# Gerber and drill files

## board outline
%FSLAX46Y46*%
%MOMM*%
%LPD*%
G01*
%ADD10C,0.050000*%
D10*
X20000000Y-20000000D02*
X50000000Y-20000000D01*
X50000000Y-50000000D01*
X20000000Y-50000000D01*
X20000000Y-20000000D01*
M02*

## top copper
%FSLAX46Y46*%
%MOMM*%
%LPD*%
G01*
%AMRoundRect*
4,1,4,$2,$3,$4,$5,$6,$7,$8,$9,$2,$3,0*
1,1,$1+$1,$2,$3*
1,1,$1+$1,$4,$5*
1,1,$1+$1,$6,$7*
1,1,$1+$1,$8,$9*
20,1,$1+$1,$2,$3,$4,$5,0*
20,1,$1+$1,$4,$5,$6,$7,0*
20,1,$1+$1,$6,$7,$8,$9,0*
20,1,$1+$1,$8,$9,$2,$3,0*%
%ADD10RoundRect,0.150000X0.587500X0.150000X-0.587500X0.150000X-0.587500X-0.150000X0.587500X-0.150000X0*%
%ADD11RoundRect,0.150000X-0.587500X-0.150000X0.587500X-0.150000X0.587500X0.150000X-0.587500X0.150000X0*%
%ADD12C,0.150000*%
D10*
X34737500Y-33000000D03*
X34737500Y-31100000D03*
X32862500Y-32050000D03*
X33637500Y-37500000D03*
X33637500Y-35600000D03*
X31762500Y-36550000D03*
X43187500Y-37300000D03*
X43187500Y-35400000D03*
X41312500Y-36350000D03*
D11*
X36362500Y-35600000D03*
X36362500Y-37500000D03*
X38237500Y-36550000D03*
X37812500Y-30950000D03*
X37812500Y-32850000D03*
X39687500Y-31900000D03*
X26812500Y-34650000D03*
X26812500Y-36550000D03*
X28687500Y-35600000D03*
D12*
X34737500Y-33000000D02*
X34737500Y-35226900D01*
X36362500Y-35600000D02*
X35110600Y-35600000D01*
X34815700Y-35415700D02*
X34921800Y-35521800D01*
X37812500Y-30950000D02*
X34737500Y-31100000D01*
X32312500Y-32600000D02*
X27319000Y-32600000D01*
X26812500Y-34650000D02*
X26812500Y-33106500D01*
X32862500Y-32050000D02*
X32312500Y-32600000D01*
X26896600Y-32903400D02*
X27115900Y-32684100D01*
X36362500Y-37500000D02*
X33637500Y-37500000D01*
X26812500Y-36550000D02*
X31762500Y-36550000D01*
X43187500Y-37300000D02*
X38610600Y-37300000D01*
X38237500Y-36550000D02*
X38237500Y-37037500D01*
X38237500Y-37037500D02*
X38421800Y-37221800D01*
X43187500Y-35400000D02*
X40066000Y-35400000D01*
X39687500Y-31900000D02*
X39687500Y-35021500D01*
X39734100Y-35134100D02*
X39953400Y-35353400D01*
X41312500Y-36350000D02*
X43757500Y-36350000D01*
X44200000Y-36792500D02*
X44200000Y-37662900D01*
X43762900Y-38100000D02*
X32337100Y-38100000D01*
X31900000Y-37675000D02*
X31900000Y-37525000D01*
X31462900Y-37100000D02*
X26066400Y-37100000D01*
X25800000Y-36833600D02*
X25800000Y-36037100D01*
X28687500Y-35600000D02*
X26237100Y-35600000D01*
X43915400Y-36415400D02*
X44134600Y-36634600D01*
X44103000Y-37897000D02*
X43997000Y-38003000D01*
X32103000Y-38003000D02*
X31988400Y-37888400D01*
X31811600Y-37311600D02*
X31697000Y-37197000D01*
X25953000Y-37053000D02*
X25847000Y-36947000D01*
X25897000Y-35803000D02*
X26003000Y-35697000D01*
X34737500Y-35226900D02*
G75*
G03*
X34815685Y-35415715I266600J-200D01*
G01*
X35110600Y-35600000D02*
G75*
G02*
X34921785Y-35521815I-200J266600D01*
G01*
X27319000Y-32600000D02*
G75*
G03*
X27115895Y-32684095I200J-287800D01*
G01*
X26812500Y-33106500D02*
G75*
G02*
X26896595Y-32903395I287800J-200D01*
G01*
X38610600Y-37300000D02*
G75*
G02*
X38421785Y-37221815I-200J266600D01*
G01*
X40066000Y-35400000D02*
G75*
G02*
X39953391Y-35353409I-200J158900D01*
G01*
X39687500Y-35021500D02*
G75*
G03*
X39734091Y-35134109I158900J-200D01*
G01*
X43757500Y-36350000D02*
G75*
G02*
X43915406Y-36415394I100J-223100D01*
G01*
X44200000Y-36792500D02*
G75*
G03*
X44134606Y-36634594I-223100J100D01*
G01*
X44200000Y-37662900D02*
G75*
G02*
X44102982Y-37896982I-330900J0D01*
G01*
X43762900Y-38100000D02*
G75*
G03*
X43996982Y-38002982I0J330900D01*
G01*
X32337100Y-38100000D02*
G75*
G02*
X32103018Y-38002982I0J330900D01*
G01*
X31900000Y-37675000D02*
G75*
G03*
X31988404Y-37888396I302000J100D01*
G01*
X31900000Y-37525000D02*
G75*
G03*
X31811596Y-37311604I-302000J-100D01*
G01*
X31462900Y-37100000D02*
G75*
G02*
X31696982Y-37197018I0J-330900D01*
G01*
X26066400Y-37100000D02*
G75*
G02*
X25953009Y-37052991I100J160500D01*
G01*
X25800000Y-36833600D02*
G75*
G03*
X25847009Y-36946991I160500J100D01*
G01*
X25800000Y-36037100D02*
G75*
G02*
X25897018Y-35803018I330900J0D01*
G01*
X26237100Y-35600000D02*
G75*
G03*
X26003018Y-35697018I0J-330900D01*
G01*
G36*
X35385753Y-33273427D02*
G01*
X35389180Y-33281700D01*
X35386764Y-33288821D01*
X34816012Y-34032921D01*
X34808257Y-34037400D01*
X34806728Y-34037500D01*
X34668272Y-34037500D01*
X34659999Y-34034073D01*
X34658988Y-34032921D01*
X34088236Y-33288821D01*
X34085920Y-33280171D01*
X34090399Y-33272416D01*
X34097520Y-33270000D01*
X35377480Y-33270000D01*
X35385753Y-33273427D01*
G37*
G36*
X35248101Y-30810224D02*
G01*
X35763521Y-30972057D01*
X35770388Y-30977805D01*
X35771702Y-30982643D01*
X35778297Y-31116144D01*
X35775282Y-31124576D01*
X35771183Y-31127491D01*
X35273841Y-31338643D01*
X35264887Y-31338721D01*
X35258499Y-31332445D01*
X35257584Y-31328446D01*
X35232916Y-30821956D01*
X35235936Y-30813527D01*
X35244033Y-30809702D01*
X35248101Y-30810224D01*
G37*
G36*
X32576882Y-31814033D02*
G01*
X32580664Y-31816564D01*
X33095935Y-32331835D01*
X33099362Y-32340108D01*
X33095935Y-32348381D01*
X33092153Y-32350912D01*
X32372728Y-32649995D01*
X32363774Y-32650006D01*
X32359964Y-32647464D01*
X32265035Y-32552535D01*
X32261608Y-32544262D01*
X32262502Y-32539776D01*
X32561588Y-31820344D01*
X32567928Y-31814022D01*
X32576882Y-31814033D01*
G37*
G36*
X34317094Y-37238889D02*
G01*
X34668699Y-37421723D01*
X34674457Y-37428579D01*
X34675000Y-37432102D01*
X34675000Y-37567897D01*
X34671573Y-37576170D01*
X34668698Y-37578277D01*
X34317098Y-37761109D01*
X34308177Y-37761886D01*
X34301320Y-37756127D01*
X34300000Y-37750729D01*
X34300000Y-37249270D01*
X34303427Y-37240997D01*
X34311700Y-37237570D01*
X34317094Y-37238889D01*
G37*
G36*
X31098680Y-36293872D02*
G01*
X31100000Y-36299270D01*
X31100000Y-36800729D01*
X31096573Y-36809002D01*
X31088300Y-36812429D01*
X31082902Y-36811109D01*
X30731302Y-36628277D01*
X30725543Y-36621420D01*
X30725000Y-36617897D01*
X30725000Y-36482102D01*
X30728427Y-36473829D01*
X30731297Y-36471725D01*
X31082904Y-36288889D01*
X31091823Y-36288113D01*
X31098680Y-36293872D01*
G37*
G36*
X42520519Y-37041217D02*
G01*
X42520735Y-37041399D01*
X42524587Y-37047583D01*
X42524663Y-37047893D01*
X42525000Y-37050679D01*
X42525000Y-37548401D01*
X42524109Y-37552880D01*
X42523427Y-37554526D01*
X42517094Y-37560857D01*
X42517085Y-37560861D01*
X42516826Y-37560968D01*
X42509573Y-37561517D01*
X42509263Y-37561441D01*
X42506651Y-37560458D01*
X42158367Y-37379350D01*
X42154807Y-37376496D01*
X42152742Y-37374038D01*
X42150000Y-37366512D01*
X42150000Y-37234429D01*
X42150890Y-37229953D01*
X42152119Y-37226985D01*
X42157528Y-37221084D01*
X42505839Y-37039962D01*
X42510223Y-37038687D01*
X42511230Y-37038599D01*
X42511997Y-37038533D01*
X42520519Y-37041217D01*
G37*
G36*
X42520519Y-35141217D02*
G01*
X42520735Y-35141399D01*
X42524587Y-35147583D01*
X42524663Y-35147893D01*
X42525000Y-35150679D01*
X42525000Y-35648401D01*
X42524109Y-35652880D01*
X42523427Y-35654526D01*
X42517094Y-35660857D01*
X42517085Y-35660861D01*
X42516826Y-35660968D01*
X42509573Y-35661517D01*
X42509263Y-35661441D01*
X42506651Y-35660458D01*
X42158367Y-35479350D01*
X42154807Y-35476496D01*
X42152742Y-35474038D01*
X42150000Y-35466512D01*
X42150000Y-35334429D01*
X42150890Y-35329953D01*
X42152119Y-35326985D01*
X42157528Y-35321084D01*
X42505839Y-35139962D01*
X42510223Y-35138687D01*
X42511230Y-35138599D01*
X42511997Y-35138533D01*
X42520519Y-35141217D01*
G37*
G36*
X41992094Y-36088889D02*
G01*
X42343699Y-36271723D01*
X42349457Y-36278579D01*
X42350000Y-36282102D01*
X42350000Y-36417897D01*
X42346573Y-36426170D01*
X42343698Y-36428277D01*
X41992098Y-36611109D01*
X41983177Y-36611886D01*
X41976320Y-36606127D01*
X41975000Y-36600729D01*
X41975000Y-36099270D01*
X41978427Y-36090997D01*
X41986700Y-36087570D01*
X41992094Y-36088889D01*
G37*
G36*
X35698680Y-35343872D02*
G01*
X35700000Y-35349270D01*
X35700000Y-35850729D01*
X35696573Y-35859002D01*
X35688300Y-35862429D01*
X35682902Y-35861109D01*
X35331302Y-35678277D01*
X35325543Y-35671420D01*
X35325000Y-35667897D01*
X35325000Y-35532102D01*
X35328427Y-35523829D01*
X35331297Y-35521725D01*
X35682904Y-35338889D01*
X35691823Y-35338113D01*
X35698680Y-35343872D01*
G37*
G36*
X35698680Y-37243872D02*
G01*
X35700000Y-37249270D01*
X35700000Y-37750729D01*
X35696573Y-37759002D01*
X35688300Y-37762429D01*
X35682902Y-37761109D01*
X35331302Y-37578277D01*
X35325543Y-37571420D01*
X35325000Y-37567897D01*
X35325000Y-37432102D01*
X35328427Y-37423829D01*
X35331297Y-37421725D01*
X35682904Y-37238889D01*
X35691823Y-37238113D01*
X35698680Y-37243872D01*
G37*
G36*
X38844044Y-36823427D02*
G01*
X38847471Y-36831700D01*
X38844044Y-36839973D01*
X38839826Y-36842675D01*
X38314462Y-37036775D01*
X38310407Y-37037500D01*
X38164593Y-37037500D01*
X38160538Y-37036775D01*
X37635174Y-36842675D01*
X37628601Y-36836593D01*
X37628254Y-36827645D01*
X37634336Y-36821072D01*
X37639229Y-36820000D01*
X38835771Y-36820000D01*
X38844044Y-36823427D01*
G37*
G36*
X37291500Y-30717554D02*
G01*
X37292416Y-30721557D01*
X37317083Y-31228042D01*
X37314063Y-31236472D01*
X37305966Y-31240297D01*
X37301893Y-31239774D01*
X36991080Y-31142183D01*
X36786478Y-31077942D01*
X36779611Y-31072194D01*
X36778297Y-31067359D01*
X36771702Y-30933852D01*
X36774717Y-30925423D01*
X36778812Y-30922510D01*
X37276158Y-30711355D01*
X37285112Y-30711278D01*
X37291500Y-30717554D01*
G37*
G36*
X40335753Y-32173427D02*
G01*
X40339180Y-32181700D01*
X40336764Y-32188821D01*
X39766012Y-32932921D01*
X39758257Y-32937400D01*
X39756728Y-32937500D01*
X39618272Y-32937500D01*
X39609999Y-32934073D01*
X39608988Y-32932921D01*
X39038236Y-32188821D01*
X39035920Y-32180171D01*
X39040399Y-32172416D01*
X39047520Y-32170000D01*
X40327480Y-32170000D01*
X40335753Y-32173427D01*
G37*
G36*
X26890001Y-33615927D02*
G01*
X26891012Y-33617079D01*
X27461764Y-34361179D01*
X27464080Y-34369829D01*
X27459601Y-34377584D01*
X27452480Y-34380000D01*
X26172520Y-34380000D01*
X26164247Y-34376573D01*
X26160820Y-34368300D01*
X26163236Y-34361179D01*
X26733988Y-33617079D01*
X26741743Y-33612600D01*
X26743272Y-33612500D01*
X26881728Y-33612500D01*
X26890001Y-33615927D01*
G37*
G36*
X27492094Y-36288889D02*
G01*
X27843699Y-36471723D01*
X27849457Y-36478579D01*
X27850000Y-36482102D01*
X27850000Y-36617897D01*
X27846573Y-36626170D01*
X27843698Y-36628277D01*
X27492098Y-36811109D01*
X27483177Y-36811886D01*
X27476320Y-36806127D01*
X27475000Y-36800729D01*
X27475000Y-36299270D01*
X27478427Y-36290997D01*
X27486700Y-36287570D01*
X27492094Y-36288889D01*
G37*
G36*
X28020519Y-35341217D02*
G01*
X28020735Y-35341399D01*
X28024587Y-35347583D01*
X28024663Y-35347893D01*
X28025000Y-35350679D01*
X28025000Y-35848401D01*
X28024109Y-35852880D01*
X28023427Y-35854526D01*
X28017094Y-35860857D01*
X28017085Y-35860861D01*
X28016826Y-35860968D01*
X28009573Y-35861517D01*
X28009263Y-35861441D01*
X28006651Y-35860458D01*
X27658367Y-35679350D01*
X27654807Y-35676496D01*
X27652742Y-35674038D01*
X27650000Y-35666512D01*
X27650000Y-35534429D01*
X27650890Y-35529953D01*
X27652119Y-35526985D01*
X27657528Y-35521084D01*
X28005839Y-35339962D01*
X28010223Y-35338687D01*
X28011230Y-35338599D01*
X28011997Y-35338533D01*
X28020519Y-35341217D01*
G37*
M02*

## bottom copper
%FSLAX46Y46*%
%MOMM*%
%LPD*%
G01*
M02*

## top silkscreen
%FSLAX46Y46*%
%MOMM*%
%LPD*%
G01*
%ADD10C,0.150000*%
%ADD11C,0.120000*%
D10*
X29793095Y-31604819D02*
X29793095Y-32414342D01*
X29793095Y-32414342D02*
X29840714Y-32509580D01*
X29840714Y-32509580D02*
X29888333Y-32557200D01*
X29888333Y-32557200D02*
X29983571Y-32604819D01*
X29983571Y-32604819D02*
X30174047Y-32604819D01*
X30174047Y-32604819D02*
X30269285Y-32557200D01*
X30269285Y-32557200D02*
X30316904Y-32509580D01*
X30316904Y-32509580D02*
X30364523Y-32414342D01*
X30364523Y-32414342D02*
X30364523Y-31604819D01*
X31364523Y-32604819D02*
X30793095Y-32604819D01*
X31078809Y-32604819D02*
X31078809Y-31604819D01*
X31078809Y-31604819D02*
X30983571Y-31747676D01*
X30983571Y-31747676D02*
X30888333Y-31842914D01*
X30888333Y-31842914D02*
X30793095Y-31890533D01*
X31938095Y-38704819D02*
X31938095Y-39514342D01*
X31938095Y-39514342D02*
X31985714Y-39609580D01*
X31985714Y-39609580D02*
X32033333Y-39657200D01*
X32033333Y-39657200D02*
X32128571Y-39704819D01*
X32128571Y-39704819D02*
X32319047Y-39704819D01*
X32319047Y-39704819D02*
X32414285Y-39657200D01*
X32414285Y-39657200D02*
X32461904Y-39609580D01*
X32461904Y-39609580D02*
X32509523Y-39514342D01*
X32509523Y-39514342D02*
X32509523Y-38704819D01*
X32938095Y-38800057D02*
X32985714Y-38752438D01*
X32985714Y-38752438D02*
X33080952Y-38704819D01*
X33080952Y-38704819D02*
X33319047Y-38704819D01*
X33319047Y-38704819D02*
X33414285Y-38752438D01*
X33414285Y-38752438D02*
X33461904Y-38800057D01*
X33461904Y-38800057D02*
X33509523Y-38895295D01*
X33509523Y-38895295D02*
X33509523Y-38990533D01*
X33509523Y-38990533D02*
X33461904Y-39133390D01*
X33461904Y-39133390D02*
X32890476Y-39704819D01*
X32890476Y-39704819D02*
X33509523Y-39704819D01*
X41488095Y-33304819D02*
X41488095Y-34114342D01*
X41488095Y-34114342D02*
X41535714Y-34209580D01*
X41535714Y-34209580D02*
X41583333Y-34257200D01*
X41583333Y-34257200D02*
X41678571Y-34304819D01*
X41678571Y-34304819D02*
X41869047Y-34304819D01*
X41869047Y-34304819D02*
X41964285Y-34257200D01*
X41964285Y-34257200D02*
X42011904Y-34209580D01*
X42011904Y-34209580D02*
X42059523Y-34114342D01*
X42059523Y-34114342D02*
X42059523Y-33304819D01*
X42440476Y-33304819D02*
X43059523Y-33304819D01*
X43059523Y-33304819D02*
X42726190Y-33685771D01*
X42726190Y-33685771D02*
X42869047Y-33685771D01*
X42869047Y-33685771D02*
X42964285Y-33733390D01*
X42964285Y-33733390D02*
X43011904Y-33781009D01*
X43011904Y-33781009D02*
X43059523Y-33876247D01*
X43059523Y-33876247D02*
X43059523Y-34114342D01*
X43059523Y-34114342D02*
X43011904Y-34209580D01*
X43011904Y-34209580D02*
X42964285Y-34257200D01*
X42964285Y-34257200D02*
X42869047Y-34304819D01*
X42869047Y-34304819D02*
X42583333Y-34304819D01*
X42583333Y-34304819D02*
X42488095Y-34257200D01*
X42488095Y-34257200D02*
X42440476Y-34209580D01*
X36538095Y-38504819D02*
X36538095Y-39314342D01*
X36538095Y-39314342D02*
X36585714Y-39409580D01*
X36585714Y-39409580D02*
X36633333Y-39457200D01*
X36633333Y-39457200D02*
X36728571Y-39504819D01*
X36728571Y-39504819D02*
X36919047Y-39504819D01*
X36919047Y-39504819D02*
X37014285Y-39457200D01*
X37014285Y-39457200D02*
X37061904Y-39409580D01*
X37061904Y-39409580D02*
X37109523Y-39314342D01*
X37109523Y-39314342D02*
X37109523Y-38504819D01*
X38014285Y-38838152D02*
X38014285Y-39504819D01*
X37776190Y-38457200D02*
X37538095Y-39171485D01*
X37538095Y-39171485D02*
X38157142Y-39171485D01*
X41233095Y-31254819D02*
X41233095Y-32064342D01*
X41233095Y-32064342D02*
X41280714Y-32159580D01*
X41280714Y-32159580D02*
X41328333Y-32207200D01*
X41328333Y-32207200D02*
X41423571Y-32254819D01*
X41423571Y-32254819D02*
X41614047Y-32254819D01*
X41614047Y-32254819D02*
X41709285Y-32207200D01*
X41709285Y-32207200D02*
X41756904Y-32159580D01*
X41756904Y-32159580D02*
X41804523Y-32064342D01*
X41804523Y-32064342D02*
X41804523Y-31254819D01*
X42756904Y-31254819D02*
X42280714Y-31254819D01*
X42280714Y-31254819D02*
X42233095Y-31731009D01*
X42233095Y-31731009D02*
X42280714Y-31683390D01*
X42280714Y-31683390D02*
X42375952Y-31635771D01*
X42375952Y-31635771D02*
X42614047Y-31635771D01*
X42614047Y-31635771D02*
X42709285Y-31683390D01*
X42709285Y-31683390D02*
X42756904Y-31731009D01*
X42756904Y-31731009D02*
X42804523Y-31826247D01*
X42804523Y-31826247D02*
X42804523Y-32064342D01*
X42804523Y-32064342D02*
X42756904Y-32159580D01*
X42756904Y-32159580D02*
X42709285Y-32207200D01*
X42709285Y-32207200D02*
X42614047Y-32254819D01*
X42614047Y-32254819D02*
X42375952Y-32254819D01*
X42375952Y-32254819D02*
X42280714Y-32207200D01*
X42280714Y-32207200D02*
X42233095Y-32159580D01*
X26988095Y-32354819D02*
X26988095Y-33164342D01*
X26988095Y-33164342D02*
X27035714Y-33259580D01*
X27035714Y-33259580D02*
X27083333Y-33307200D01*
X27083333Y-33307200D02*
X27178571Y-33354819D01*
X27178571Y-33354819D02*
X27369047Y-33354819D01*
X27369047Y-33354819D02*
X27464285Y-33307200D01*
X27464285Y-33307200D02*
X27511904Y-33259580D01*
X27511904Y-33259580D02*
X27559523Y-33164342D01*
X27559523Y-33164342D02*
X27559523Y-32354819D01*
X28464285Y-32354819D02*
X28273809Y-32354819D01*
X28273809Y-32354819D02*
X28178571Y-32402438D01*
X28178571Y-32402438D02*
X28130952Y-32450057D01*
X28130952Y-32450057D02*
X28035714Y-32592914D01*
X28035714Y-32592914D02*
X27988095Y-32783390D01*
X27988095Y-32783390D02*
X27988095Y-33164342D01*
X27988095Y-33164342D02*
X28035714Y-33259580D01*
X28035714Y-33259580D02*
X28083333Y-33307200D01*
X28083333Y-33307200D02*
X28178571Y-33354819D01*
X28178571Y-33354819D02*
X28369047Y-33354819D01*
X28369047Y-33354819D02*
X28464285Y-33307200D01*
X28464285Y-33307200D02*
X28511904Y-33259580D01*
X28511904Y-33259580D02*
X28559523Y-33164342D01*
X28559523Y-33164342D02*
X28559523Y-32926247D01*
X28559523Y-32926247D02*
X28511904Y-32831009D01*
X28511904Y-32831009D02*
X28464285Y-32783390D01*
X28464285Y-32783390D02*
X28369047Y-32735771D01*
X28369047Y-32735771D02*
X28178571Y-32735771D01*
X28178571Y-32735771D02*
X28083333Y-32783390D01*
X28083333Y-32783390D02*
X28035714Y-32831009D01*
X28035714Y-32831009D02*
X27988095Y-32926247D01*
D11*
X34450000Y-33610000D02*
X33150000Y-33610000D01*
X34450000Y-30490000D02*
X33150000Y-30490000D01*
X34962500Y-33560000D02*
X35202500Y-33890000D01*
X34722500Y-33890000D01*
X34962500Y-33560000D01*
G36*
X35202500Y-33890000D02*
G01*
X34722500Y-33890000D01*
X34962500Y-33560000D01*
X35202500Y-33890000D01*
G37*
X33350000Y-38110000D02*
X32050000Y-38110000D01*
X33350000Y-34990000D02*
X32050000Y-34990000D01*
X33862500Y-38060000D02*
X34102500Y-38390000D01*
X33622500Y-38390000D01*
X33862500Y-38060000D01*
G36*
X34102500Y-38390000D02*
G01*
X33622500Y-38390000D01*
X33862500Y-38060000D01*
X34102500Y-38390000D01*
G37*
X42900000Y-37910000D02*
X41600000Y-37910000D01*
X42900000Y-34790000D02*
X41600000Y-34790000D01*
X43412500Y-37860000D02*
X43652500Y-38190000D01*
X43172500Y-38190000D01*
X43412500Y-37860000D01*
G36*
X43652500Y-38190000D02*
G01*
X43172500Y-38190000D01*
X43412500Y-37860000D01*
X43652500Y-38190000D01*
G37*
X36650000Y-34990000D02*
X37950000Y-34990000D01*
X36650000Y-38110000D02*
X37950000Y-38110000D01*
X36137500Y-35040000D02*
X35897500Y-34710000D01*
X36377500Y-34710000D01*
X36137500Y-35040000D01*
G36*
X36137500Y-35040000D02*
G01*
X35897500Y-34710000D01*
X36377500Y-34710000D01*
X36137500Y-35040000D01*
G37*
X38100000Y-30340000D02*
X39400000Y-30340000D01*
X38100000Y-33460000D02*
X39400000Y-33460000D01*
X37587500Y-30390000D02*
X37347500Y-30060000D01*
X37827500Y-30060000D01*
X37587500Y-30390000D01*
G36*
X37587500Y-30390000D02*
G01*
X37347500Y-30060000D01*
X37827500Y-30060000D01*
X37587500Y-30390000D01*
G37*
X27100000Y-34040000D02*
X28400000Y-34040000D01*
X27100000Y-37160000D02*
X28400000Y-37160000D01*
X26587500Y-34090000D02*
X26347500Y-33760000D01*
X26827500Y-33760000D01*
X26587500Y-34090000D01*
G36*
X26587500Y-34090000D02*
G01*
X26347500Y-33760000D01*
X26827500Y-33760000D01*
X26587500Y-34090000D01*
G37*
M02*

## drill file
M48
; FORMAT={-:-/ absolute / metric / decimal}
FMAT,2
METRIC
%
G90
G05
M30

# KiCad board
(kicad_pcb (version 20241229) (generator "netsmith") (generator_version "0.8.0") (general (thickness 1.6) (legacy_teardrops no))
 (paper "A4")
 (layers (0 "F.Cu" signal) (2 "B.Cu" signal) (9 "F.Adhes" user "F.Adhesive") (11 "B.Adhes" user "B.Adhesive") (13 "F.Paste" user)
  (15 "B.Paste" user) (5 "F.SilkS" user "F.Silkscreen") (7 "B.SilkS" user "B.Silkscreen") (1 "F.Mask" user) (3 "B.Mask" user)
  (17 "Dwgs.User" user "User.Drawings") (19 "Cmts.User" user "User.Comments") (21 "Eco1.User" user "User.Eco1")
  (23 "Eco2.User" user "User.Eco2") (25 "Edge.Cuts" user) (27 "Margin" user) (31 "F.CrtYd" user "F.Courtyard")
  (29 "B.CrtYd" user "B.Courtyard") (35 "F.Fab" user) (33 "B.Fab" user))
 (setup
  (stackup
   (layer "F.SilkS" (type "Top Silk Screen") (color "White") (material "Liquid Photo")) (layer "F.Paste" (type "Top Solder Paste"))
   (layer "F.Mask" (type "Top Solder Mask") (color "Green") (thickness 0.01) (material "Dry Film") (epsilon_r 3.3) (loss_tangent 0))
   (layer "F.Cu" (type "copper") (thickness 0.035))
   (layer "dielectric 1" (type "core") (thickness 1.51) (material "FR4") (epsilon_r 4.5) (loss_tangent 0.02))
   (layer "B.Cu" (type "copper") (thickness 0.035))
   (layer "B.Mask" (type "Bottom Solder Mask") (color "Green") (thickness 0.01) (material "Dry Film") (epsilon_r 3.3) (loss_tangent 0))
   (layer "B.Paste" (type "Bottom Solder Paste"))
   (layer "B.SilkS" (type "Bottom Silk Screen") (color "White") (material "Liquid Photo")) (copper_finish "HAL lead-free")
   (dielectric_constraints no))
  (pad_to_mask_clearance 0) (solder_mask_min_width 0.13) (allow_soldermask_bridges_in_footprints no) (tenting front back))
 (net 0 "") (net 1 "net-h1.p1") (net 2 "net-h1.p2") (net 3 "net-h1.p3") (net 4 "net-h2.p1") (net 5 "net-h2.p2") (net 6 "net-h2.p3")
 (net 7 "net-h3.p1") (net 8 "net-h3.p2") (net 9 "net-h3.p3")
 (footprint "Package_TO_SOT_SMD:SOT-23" (layer "F.Cu") (at 33.8 32.05 180)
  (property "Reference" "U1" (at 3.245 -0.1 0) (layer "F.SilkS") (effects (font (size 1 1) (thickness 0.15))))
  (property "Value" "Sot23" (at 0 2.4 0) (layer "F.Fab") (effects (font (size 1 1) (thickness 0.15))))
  (pad "1" smd roundrect (at -0.9375 -0.95 180) (size 1.475 0.6) (layers "F.Cu" "F.Mask" "F.Paste") (roundrect_rratio 0.25)
   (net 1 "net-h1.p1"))
  (pad "2" smd roundrect (at -0.9375 0.95 180) (size 1.475 0.6) (layers "F.Cu" "F.Mask" "F.Paste") (roundrect_rratio 0.25)
   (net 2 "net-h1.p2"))
  (pad "3" smd roundrect (at 0.9375 0 180) (size 1.475 0.6) (layers "F.Cu" "F.Mask" "F.Paste") (roundrect_rratio 0.25) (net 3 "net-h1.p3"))
  (fp_line (start -0.65 -1.56) (end 0.65 -1.56) (stroke (width 0.12) (type solid)) (layer "F.SilkS"))
  (fp_line (start -0.65 1.56) (end 0.65 1.56) (stroke (width 0.12) (type solid)) (layer "F.SilkS"))
  (fp_poly (pts (xy -1.1625 -1.51) (xy -1.4025 -1.84) (xy -0.9225 -1.84)) (stroke (width 0.12) (type solid)) (fill solid) (layer "F.SilkS")))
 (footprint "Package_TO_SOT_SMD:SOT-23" (layer "F.Cu") (at 32.7 36.55 180)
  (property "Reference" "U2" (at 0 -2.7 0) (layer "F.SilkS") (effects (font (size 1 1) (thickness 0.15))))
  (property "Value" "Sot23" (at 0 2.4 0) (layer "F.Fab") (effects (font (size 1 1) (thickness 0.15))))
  (pad "1" smd roundrect (at -0.9375 -0.95 180) (size 1.475 0.6) (layers "F.Cu" "F.Mask" "F.Paste") (roundrect_rratio 0.25)
   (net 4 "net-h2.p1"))
  (pad "2" smd roundrect (at -0.9375 0.95 180) (size 1.475 0.6) (layers "F.Cu" "F.Mask" "F.Paste") (roundrect_rratio 0.25)
   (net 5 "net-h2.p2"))
  (pad "3" smd roundrect (at 0.9375 0 180) (size 1.475 0.6) (layers "F.Cu" "F.Mask" "F.Paste") (roundrect_rratio 0.25) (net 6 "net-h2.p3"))
  (fp_line (start -0.65 -1.56) (end 0.65 -1.56) (stroke (width 0.12) (type solid)) (layer "F.SilkS"))
  (fp_line (start -0.65 1.56) (end 0.65 1.56) (stroke (width 0.12) (type solid)) (layer "F.SilkS"))
  (fp_poly (pts (xy -1.1625 -1.51) (xy -1.4025 -1.84) (xy -0.9225 -1.84)) (stroke (width 0.12) (type solid)) (fill solid) (layer "F.SilkS")))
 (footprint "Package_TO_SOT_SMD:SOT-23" (layer "F.Cu") (at 42.25 36.35 180)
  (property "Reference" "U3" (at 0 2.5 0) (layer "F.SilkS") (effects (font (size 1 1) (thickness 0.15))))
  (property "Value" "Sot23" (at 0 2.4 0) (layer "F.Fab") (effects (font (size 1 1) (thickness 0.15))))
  (pad "1" smd roundrect (at -0.9375 -0.95 180) (size 1.475 0.6) (layers "F.Cu" "F.Mask" "F.Paste") (roundrect_rratio 0.25)
   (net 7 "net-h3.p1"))
  (pad "2" smd roundrect (at -0.9375 0.95 180) (size 1.475 0.6) (layers "F.Cu" "F.Mask" "F.Paste") (roundrect_rratio 0.25)
   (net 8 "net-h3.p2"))
  (pad "3" smd roundrect (at 0.9375 0 180) (size 1.475 0.6) (layers "F.Cu" "F.Mask" "F.Paste") (roundrect_rratio 0.25) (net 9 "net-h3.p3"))
  (fp_line (start -0.65 -1.56) (end 0.65 -1.56) (stroke (width 0.12) (type solid)) (layer "F.SilkS"))
  (fp_line (start -0.65 1.56) (end 0.65 1.56) (stroke (width 0.12) (type solid)) (layer "F.SilkS"))
  (fp_poly (pts (xy -1.1625 -1.51) (xy -1.4025 -1.84) (xy -0.9225 -1.84)) (stroke (width 0.12) (type solid)) (fill solid) (layer "F.SilkS")))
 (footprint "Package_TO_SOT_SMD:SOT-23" (layer "F.Cu") (at 37.3 36.55)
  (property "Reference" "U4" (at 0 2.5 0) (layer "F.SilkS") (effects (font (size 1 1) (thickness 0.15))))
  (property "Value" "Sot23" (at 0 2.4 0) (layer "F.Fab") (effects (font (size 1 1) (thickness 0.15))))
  (pad "1" smd roundrect (at -0.9375 -0.95) (size 1.475 0.6) (layers "F.Cu" "F.Mask" "F.Paste") (roundrect_rratio 0.25) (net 1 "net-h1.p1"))
  (pad "2" smd roundrect (at -0.9375 0.95) (size 1.475 0.6) (layers "F.Cu" "F.Mask" "F.Paste") (roundrect_rratio 0.25) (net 4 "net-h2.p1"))
  (pad "3" smd roundrect (at 0.9375 0) (size 1.475 0.6) (layers "F.Cu" "F.Mask" "F.Paste") (roundrect_rratio 0.25) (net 7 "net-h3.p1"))
  (fp_line (start -0.65 -1.56) (end 0.65 -1.56) (stroke (width 0.12) (type solid)) (layer "F.SilkS"))
  (fp_line (start -0.65 1.56) (end 0.65 1.56) (stroke (width 0.12) (type solid)) (layer "F.SilkS"))
  (fp_poly (pts (xy -1.1625 -1.51) (xy -1.4025 -1.84) (xy -0.9225 -1.84)) (stroke (width 0.12) (type solid)) (fill solid) (layer "F.SilkS")))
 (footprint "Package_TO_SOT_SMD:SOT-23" (layer "F.Cu") (at 38.75 31.9)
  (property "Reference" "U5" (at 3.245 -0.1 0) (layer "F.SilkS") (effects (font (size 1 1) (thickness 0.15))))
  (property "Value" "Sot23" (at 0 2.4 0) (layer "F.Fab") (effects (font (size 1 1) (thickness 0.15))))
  (pad "1" smd roundrect (at -0.9375 -0.95) (size 1.475 0.6) (layers "F.Cu" "F.Mask" "F.Paste") (roundrect_rratio 0.25) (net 2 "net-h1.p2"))
  (pad "2" smd roundrect (at -0.9375 0.95) (size 1.475 0.6) (layers "F.Cu" "F.Mask" "F.Paste") (roundrect_rratio 0.25) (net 5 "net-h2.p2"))
  (pad "3" smd roundrect (at 0.9375 0) (size 1.475 0.6) (layers "F.Cu" "F.Mask" "F.Paste") (roundrect_rratio 0.25) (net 8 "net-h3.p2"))
  (fp_line (start -0.65 -1.56) (end 0.65 -1.56) (stroke (width 0.12) (type solid)) (layer "F.SilkS"))
  (fp_line (start -0.65 1.56) (end 0.65 1.56) (stroke (width 0.12) (type solid)) (layer "F.SilkS"))
  (fp_poly (pts (xy -1.1625 -1.51) (xy -1.4025 -1.84) (xy -0.9225 -1.84)) (stroke (width 0.12) (type solid)) (fill solid) (layer "F.SilkS")))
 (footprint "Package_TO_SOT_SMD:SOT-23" (layer "F.Cu") (at 27.75 35.6)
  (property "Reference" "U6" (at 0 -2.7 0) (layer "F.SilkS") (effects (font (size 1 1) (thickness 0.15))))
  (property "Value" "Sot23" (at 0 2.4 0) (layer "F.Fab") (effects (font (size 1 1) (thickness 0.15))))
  (pad "1" smd roundrect (at -0.9375 -0.95) (size 1.475 0.6) (layers "F.Cu" "F.Mask" "F.Paste") (roundrect_rratio 0.25) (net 3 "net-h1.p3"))
  (pad "2" smd roundrect (at -0.9375 0.95) (size 1.475 0.6) (layers "F.Cu" "F.Mask" "F.Paste") (roundrect_rratio 0.25) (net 6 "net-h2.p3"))
  (pad "3" smd roundrect (at 0.9375 0) (size 1.475 0.6) (layers "F.Cu" "F.Mask" "F.Paste") (roundrect_rratio 0.25) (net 9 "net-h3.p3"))
  (fp_line (start -0.65 -1.56) (end 0.65 -1.56) (stroke (width 0.12) (type solid)) (layer "F.SilkS"))
  (fp_line (start -0.65 1.56) (end 0.65 1.56) (stroke (width 0.12) (type solid)) (layer "F.SilkS"))
  (fp_poly (pts (xy -1.1625 -1.51) (xy -1.4025 -1.84) (xy -0.9225 -1.84)) (stroke (width 0.12) (type solid)) (fill solid) (layer "F.SilkS")))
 (segment (start 34.7375 33) (end 34.7375 35.2269) (width 0.15) (layer "F.Cu") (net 1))
 (segment (start 36.3625 35.6) (end 35.1106 35.6) (width 0.15) (layer "F.Cu") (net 1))
 (segment (start 34.8157 35.4157) (end 34.9218 35.5218) (width 0.15) (layer "F.Cu") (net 1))
 (segment (start 37.8125 30.95) (end 34.7375 31.1) (width 0.15) (layer "F.Cu") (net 2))
 (segment (start 32.3125 32.6) (end 27.319 32.6) (width 0.15) (layer "F.Cu") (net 3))
 (segment (start 26.8125 34.65) (end 26.8125 33.1065) (width 0.15) (layer "F.Cu") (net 3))
 (segment (start 32.8625 32.05) (end 32.3125 32.6) (width 0.15) (layer "F.Cu") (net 3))
 (segment (start 26.8966 32.9034) (end 27.1159 32.6841) (width 0.15) (layer "F.Cu") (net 3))
 (segment (start 36.3625 37.5) (end 33.6375 37.5) (width 0.15) (layer "F.Cu") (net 4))
 (segment (start 26.8125 36.55) (end 31.7625 36.55) (width 0.15) (layer "F.Cu") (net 6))
 (segment (start 43.1875 37.3) (end 38.6106 37.3) (width 0.15) (layer "F.Cu") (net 7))
 (segment (start 38.2375 36.55) (end 38.2375 37.0375) (width 0.15) (layer "F.Cu") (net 7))
 (segment (start 38.2375 37.0375) (end 38.4218 37.2218) (width 0.15) (layer "F.Cu") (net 7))
 (segment (start 43.1875 35.4) (end 40.066 35.4) (width 0.15) (layer "F.Cu") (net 8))
 (segment (start 39.6875 31.9) (end 39.6875 35.0215) (width 0.15) (layer "F.Cu") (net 8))
 (segment (start 39.7341 35.1341) (end 39.9534 35.3534) (width 0.15) (layer "F.Cu") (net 8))
 (segment (start 41.3125 36.35) (end 43.7575 36.35) (width 0.15) (layer "F.Cu") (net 9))
 (segment (start 44.2 36.7925) (end 44.2 37.6629) (width 0.15) (layer "F.Cu") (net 9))
 (segment (start 43.7629 38.1) (end 32.3371 38.1) (width 0.15) (layer "F.Cu") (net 9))
 (segment (start 31.9 37.675) (end 31.9 37.525) (width 0.15) (layer "F.Cu") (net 9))
 (segment (start 31.4629 37.1) (end 26.0664 37.1) (width 0.15) (layer "F.Cu") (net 9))
 (segment (start 25.8 36.8336) (end 25.8 36.0371) (width 0.15) (layer "F.Cu") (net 9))
 (segment (start 28.6875 35.6) (end 26.2371 35.6) (width 0.15) (layer "F.Cu") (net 9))
 (segment (start 43.9154 36.4154) (end 44.1346 36.6346) (width 0.15) (layer "F.Cu") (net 9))
 (segment (start 44.103 37.897) (end 43.997 38.003) (width 0.15) (layer "F.Cu") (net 9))
 (segment (start 32.103 38.003) (end 31.9884 37.8884) (width 0.15) (layer "F.Cu") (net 9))
 (segment (start 31.8116 37.3116) (end 31.697 37.197) (width 0.15) (layer "F.Cu") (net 9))
 (segment (start 25.953 37.053) (end 25.847 36.947) (width 0.15) (layer "F.Cu") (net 9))
 (segment (start 25.897 35.803) (end 26.003 35.697) (width 0.15) (layer "F.Cu") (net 9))
 (arc (start 34.7375 35.2269) (mid 34.7578 35.3291) (end 34.8157 35.4157) (width 0.15) (layer "F.Cu") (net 1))
 (arc (start 35.1106 35.6) (mid 35.0084 35.5797) (end 34.9218 35.5218) (width 0.15) (layer "F.Cu") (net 1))
 (arc (start 27.319 32.6) (mid 27.2091 32.6219) (end 27.1159 32.6841) (width 0.15) (layer "F.Cu") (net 3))
 (arc (start 26.8125 33.1065) (mid 26.8344 32.9966) (end 26.8966 32.9034) (width 0.15) (layer "F.Cu") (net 3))
 (arc (start 38.6106 37.3) (mid 38.5084 37.2797) (end 38.4218 37.2218) (width 0.15) (layer "F.Cu") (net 7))
 (arc (start 40.066 35.4) (mid 40.005 35.3879) (end 39.9534 35.3534) (width 0.15) (layer "F.Cu") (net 8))
 (arc (start 39.6875 35.0215) (mid 39.6996 35.0825) (end 39.7341 35.1341) (width 0.15) (layer "F.Cu") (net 8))
 (arc (start 43.7575 36.35) (mid 43.843 36.367) (end 43.9154 36.4154) (width 0.15) (layer "F.Cu") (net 9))
 (arc (start 44.2 36.7925) (mid 44.183 36.707) (end 44.1346 36.6346) (width 0.15) (layer "F.Cu") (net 9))
 (arc (start 44.2 37.6629) (mid 44.1748 37.7896) (end 44.103 37.897) (width 0.15) (layer "F.Cu") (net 9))
 (arc (start 43.7629 38.1) (mid 43.8896 38.0748) (end 43.997 38.003) (width 0.15) (layer "F.Cu") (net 9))
 (arc (start 32.3371 38.1) (mid 32.2104 38.0748) (end 32.103 38.003) (width 0.15) (layer "F.Cu") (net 9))
 (arc (start 31.9 37.675) (mid 31.923 37.7905) (end 31.9884 37.8884) (width 0.15) (layer "F.Cu") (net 9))
 (arc (start 31.9 37.525) (mid 31.877 37.4095) (end 31.8116 37.3116) (width 0.15) (layer "F.Cu") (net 9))
 (arc (start 31.4629 37.1) (mid 31.5896 37.1252) (end 31.697 37.197) (width 0.15) (layer "F.Cu") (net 9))
 (arc (start 26.0664 37.1) (mid 26.0051 37.0878) (end 25.953 37.053) (width 0.15) (layer "F.Cu") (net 9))
 (arc (start 25.8 36.8336) (mid 25.8122 36.8949) (end 25.847 36.947) (width 0.15) (layer "F.Cu") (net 9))
 (arc (start 25.8 36.0371) (mid 25.8252 35.9104) (end 25.897 35.803) (width 0.15) (layer "F.Cu") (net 9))
 (arc (start 26.2371 35.6) (mid 26.1104 35.6252) (end 26.003 35.697) (width 0.15) (layer "F.Cu") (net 9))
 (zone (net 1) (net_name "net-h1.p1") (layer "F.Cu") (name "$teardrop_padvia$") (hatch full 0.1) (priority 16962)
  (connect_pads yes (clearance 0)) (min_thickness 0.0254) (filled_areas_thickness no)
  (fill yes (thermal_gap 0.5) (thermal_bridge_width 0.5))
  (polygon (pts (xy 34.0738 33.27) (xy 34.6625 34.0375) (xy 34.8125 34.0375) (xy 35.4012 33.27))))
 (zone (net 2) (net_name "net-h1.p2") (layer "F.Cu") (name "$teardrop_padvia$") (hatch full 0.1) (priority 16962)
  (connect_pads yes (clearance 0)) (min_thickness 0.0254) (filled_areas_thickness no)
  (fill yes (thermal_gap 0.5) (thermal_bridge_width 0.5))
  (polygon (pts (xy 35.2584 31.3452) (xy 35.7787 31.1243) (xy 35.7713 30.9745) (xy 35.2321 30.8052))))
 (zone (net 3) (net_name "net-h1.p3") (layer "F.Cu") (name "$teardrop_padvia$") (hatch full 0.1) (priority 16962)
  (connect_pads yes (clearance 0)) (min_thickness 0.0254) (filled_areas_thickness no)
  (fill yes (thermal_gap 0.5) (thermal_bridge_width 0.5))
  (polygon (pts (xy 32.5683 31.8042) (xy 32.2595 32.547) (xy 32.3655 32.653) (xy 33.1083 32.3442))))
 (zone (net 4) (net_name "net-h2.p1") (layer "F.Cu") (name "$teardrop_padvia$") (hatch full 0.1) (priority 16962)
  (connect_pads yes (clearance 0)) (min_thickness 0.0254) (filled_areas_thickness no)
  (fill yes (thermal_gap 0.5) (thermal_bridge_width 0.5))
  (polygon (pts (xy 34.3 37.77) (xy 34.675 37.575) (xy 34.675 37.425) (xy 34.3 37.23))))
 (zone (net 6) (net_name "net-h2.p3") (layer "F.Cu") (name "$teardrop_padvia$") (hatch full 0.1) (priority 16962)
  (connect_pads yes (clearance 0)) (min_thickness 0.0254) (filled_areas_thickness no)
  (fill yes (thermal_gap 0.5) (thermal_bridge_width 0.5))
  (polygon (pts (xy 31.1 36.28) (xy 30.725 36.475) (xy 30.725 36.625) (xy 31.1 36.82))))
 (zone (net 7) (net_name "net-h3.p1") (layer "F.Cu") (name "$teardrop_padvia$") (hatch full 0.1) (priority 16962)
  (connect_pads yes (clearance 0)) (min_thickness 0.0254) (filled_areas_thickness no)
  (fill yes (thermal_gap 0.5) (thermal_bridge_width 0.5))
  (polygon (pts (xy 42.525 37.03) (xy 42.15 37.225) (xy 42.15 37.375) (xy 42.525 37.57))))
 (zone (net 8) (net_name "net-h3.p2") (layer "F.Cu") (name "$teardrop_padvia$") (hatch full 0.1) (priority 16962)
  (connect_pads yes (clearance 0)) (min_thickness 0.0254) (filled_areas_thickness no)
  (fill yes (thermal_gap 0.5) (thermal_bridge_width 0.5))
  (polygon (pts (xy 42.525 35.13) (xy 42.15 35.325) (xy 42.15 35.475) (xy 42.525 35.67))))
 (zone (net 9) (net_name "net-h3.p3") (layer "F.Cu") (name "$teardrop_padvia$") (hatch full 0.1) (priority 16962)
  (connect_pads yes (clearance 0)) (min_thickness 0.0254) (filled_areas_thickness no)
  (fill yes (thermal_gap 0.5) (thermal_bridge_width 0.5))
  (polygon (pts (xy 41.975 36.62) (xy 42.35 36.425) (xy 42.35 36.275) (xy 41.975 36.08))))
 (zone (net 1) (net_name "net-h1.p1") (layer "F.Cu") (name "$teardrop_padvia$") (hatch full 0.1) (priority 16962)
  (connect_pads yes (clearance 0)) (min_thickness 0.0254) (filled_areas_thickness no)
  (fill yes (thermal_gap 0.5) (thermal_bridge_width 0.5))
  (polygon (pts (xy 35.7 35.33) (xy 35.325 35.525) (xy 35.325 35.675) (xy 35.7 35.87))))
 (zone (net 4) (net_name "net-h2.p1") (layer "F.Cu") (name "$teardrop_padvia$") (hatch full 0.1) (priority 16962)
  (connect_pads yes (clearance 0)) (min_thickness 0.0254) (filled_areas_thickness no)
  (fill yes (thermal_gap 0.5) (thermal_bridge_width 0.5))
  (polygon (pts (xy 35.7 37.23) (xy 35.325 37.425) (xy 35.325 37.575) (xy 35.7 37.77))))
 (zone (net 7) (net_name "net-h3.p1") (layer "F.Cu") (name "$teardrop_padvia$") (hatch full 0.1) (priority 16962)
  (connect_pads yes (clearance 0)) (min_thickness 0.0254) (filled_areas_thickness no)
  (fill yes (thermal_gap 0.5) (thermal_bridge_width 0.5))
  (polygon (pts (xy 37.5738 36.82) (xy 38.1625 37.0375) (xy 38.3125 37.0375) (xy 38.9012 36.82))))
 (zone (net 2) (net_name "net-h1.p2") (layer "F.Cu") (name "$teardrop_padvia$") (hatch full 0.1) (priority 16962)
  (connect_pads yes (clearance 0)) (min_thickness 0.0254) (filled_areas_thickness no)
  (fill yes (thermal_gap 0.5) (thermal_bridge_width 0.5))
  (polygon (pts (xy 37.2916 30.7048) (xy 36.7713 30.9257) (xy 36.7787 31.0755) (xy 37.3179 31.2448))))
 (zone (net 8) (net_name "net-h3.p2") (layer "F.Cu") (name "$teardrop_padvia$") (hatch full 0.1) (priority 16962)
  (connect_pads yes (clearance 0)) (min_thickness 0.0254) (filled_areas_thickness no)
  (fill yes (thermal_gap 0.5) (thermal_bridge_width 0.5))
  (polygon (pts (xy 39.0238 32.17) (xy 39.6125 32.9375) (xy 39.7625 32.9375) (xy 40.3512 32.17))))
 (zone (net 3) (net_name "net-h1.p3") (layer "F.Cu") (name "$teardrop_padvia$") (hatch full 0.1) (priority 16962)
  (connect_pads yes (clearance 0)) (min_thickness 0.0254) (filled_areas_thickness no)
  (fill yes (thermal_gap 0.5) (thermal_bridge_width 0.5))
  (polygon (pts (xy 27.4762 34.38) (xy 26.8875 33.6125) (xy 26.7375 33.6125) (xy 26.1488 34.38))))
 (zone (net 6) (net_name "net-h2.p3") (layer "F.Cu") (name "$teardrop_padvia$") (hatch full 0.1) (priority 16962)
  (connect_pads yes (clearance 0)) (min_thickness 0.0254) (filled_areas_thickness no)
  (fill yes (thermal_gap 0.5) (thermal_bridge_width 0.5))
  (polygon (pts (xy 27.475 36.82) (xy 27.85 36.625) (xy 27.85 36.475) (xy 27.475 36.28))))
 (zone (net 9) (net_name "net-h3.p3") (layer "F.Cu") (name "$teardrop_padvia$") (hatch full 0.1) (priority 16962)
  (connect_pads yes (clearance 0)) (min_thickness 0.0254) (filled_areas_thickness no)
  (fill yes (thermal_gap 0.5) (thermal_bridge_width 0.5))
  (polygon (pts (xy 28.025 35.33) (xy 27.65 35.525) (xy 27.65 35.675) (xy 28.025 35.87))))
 (gr_rect (start 20 20) (end 50 50) (stroke (width 0.05) (type default)) (fill no) (layer "Edge.Cuts")))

